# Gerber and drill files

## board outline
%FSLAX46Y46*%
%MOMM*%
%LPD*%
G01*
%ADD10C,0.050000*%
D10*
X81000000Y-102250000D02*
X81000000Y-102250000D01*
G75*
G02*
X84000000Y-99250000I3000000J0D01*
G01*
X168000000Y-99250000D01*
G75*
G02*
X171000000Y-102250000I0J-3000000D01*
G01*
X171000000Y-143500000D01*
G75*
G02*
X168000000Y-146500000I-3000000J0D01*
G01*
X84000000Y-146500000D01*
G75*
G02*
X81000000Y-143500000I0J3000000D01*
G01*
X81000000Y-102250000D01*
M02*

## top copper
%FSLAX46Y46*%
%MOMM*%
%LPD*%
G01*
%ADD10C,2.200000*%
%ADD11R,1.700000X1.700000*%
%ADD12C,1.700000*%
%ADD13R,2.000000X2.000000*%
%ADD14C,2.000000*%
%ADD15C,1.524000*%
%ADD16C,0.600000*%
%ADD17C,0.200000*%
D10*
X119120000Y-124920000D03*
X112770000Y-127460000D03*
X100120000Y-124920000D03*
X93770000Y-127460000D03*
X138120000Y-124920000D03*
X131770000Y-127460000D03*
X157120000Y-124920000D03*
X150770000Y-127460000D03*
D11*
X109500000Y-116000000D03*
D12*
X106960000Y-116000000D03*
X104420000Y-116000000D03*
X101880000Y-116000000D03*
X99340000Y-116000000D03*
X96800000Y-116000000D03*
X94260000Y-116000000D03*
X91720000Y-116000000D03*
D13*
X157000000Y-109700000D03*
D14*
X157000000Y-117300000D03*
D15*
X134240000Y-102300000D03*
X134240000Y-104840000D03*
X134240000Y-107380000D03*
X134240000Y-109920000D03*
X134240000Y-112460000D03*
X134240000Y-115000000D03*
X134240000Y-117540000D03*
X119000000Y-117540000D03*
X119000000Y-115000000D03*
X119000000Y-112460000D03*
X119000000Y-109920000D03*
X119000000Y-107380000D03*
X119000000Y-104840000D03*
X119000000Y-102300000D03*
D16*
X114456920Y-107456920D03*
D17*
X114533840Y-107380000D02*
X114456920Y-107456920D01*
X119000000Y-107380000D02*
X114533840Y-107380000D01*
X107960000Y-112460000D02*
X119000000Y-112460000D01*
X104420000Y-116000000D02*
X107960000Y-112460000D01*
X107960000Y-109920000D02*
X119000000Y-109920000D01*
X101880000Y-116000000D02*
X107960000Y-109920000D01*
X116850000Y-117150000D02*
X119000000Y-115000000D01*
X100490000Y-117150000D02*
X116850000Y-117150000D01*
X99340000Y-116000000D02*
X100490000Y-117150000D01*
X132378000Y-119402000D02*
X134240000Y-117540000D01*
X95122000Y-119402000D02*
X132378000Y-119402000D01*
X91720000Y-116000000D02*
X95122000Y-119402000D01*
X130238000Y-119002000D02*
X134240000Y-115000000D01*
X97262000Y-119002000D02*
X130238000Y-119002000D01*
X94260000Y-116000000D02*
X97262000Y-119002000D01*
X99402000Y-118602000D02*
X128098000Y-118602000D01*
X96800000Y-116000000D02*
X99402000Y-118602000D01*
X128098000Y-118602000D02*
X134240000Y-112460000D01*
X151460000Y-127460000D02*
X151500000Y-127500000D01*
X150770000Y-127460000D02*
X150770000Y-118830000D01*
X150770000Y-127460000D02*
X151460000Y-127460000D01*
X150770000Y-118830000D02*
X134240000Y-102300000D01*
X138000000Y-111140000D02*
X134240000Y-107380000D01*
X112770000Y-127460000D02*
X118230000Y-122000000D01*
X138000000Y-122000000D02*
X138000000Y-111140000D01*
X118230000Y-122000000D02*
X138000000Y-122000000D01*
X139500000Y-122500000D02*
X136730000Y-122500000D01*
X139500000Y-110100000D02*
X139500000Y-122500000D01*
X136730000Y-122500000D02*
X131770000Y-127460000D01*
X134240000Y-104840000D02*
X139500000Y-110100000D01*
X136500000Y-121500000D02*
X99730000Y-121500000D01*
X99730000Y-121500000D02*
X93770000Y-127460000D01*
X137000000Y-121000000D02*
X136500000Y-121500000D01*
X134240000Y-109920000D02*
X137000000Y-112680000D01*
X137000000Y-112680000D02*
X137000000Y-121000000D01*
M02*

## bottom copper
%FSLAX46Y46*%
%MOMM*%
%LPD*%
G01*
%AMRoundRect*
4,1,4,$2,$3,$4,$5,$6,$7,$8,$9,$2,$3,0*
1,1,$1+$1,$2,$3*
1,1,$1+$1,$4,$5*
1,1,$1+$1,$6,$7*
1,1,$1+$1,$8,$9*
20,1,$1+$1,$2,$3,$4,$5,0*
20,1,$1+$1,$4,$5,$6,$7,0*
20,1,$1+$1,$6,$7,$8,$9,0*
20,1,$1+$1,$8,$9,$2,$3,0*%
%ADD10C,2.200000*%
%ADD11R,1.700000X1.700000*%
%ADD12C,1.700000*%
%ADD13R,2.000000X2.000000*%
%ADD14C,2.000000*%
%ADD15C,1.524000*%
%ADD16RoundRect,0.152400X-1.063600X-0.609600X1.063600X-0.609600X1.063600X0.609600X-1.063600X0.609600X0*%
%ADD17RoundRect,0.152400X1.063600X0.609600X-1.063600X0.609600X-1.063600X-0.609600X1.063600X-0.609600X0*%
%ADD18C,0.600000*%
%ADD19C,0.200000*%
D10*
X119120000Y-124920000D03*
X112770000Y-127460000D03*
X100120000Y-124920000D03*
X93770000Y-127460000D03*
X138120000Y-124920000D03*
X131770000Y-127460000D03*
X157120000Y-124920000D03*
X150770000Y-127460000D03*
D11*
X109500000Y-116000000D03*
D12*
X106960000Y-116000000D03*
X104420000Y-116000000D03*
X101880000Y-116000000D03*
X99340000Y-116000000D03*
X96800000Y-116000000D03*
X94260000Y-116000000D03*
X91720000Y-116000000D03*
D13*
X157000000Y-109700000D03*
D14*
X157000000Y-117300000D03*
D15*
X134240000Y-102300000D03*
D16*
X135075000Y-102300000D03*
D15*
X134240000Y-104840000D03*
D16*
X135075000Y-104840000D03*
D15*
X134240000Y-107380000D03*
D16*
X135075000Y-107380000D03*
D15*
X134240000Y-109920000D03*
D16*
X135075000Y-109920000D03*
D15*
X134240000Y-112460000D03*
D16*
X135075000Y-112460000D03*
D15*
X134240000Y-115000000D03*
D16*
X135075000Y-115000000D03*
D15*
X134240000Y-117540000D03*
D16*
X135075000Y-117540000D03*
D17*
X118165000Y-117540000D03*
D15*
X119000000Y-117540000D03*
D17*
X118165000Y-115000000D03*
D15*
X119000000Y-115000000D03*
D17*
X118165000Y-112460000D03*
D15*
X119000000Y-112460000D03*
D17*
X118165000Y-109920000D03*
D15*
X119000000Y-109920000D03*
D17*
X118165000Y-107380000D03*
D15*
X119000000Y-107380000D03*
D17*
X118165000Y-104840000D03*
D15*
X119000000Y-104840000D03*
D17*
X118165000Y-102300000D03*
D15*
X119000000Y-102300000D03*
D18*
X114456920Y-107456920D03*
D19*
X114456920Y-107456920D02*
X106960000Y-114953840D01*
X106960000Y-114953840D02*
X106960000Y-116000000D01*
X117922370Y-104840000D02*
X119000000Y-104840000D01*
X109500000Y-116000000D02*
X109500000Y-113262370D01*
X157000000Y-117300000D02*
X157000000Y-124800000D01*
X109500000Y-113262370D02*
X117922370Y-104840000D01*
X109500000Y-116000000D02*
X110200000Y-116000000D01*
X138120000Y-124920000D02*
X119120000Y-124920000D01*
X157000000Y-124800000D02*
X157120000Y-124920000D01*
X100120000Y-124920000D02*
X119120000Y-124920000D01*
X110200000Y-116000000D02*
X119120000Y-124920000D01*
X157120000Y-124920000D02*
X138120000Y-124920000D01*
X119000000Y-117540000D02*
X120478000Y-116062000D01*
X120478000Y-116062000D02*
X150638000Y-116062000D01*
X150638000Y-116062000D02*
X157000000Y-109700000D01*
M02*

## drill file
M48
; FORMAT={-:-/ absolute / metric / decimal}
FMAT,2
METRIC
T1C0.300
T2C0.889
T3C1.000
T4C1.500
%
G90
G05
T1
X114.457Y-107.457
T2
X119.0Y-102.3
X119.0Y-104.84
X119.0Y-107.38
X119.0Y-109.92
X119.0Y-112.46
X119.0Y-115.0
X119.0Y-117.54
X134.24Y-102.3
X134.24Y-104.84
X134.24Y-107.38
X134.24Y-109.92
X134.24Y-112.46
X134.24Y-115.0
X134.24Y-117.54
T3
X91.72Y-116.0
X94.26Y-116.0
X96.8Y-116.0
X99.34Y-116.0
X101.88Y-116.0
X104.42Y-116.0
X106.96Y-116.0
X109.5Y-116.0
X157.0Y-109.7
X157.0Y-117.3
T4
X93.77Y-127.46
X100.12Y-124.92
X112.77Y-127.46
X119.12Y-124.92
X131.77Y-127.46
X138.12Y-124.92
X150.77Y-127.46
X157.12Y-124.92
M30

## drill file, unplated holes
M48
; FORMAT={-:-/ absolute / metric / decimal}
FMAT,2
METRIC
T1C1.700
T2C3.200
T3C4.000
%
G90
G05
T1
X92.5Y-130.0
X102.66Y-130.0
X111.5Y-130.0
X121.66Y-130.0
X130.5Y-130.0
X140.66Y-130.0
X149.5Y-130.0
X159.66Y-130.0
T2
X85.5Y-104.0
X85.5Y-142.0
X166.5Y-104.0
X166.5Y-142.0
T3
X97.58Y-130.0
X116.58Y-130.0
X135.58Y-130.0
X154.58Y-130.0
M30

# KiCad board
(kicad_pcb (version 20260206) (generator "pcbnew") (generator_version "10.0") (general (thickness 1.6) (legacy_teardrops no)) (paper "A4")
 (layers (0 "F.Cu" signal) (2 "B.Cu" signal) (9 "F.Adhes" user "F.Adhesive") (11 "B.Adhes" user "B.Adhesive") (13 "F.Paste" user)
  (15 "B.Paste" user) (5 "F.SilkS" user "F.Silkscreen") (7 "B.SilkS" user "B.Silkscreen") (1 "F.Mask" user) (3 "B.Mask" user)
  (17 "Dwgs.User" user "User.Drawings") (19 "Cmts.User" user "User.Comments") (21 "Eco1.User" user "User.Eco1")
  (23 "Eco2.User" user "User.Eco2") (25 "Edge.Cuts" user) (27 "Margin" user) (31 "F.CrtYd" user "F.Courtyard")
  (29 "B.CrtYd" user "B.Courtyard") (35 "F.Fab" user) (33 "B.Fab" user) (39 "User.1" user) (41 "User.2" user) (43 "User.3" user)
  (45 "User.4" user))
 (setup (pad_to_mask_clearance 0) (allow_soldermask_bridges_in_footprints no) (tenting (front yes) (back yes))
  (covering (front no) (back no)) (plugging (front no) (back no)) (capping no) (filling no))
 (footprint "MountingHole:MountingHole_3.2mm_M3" (layer "F.Cu") (at 85.5 104)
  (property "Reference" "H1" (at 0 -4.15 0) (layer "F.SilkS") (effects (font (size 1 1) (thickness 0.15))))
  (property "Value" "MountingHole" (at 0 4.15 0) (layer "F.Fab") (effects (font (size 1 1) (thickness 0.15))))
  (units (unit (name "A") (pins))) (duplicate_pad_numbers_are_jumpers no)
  (pad "" np_thru_hole circle (at 0 0) (size 3.2 3.2) (drill 3.2) (layers "*.Cu" "*.Mask")))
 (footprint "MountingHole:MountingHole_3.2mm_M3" (layer "F.Cu") (at 85.5 142)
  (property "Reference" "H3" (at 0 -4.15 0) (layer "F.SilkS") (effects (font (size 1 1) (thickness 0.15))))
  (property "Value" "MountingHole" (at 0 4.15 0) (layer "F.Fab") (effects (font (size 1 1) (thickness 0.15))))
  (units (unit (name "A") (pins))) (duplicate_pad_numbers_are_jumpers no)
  (pad "" np_thru_hole circle (at 0 0) (size 3.2 3.2) (drill 3.2) (layers "*.Cu" "*.Mask")))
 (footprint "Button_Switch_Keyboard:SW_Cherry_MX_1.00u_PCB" (layer "F.Cu") (at 119.12 124.92)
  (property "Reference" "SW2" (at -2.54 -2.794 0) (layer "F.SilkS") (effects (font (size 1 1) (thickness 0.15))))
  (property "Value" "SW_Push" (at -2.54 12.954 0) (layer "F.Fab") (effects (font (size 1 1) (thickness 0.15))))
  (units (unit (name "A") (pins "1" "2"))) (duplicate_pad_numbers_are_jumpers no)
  (pad "" np_thru_hole circle (at -7.62 5.08) (size 1.7 1.7) (drill 1.7) (layers "*.Cu" "*.Mask"))
  (pad "" np_thru_hole circle (at -2.54 5.08) (size 4 4) (drill 4) (layers "*.Cu" "*.Mask"))
  (pad "" np_thru_hole circle (at 2.54 5.08) (size 1.7 1.7) (drill 1.7) (layers "*.Cu" "*.Mask"))
  (pad "1" thru_hole circle (at 0 0) (size 2.2 2.2) (drill 1.5) (layers "*.Cu" "*.Mask") (remove_unused_layers no) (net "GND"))
  (pad "2" thru_hole circle (at -6.35 2.54) (size 2.2 2.2) (drill 1.5) (layers "*.Cu" "*.Mask") (remove_unused_layers no)
   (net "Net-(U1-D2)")))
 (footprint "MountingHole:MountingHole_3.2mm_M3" (layer "F.Cu") (at 166.5 142)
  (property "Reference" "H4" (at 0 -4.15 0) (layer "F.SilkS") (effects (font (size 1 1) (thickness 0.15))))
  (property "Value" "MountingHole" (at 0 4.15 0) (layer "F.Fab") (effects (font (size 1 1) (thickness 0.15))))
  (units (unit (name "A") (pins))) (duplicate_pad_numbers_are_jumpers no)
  (pad "" np_thru_hole circle (at 0 0) (size 3.2 3.2) (drill 3.2) (layers "*.Cu" "*.Mask")))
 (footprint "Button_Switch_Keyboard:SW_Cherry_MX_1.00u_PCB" (layer "F.Cu") (at 100.12 124.92)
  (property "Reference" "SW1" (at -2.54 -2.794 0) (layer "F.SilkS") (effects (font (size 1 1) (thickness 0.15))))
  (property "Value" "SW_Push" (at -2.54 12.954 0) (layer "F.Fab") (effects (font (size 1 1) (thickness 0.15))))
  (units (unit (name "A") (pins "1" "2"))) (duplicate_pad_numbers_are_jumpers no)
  (pad "" np_thru_hole circle (at -7.62 5.08) (size 1.7 1.7) (drill 1.7) (layers "*.Cu" "*.Mask"))
  (pad "" np_thru_hole circle (at -2.54 5.08) (size 4 4) (drill 4) (layers "*.Cu" "*.Mask"))
  (pad "" np_thru_hole circle (at 2.54 5.08) (size 1.7 1.7) (drill 1.7) (layers "*.Cu" "*.Mask"))
  (pad "1" thru_hole circle (at 0 0) (size 2.2 2.2) (drill 1.5) (layers "*.Cu" "*.Mask") (remove_unused_layers no) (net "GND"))
  (pad "2" thru_hole circle (at -6.35 2.54) (size 2.2 2.2) (drill 1.5) (layers "*.Cu" "*.Mask") (remove_unused_layers no)
   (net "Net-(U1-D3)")))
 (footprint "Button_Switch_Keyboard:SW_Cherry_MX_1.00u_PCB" (layer "F.Cu") (at 138.12 124.92)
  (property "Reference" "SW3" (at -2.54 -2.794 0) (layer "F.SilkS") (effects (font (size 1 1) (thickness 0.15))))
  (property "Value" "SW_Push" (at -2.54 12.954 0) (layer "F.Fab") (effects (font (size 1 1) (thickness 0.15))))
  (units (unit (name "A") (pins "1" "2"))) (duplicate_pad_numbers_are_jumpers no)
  (pad "" np_thru_hole circle (at -7.62 5.08) (size 1.7 1.7) (drill 1.7) (layers "*.Cu" "*.Mask"))
  (pad "" np_thru_hole circle (at -2.54 5.08) (size 4 4) (drill 4) (layers "*.Cu" "*.Mask"))
  (pad "" np_thru_hole circle (at 2.54 5.08) (size 1.7 1.7) (drill 1.7) (layers "*.Cu" "*.Mask"))
  (pad "1" thru_hole circle (at 0 0) (size 2.2 2.2) (drill 1.5) (layers "*.Cu" "*.Mask") (remove_unused_layers no) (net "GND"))
  (pad "2" thru_hole circle (at -6.35 2.54) (size 2.2 2.2) (drill 1.5) (layers "*.Cu" "*.Mask") (remove_unused_layers no)
   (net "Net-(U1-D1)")))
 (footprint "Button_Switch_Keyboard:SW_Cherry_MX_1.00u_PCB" (layer "F.Cu") (at 157.12 124.92)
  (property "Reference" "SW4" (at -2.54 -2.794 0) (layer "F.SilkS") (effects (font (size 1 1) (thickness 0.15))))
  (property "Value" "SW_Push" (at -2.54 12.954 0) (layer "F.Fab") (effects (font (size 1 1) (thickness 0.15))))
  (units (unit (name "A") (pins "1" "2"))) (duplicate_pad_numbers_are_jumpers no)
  (pad "" np_thru_hole circle (at -7.62 5.08) (size 1.7 1.7) (drill 1.7) (layers "*.Cu" "*.Mask"))
  (pad "" np_thru_hole circle (at -2.54 5.08) (size 4 4) (drill 4) (layers "*.Cu" "*.Mask"))
  (pad "" np_thru_hole circle (at 2.54 5.08) (size 1.7 1.7) (drill 1.7) (layers "*.Cu" "*.Mask"))
  (pad "1" thru_hole circle (at 0 0) (size 2.2 2.2) (drill 1.5) (layers "*.Cu" "*.Mask") (remove_unused_layers no) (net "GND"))
  (pad "2" thru_hole circle (at -6.35 2.54) (size 2.2 2.2) (drill 1.5) (layers "*.Cu" "*.Mask") (remove_unused_layers no)
   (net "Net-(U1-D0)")))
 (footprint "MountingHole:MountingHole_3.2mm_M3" (layer "F.Cu") (at 166.5 104)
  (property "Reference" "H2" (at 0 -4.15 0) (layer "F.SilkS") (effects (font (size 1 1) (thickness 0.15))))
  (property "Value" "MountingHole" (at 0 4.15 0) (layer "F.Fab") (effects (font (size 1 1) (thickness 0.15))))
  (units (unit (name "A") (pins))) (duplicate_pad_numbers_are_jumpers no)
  (pad "" np_thru_hole circle (at 0 0) (size 3.2 3.2) (drill 3.2) (layers "*.Cu" "*.Mask")))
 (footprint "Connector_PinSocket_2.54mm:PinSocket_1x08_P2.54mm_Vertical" (layer "B.Cu") (at 109.5 116 90)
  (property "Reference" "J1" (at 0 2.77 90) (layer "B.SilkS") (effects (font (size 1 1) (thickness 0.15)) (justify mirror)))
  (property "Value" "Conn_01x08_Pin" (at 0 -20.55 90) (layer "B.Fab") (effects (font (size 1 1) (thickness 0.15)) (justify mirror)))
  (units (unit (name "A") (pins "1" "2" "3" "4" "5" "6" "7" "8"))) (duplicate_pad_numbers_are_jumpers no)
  (pad "1" thru_hole rect (at 0 0 90) (size 1.7 1.7) (drill 1) (layers "*.Cu" "*.Mask") (remove_unused_layers no) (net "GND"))
  (pad "2" thru_hole circle (at 0 -2.54 90) (size 1.7 1.7) (drill 1) (layers "*.Cu" "*.Mask") (remove_unused_layers no) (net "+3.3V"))
  (pad "3" thru_hole circle (at 0 -5.08 90) (size 1.7 1.7) (drill 1) (layers "*.Cu" "*.Mask") (remove_unused_layers no) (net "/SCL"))
  (pad "4" thru_hole circle (at 0 -7.62 90) (size 1.7 1.7) (drill 1) (layers "*.Cu" "*.Mask") (remove_unused_layers no) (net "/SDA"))
  (pad "5" thru_hole circle (at 0 -10.16 90) (size 1.7 1.7) (drill 1) (layers "*.Cu" "*.Mask") (remove_unused_layers no) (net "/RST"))
  (pad "6" thru_hole circle (at 0 -12.7 90) (size 1.7 1.7) (drill 1) (layers "*.Cu" "*.Mask") (remove_unused_layers no) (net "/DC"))
  (pad "7" thru_hole circle (at 0 -15.24 90) (size 1.7 1.7) (drill 1) (layers "*.Cu" "*.Mask") (remove_unused_layers no) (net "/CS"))
  (pad "8" thru_hole circle (at 0 -17.78 90) (size 1.7 1.7) (drill 1) (layers "*.Cu" "*.Mask") (remove_unused_layers no) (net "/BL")))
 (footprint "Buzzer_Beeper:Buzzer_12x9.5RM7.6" (layer "B.Cu") (at 157 109.7 -90)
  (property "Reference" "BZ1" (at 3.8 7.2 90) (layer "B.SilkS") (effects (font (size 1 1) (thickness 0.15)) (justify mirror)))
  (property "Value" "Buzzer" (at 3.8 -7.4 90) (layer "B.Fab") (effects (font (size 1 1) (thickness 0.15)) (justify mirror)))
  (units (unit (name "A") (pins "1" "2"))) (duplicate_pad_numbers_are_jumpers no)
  (pad "1" thru_hole rect (at 0 0 270) (size 2 2) (drill 1) (layers "*.Cu" "*.Mask") (remove_unused_layers no) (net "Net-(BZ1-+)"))
  (pad "2" thru_hole circle (at 7.6 0 270) (size 2 2) (drill 1) (layers "*.Cu" "*.Mask") (remove_unused_layers no) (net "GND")))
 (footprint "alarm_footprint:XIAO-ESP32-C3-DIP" (layer "B.Cu") (at 126.62 109.92 90)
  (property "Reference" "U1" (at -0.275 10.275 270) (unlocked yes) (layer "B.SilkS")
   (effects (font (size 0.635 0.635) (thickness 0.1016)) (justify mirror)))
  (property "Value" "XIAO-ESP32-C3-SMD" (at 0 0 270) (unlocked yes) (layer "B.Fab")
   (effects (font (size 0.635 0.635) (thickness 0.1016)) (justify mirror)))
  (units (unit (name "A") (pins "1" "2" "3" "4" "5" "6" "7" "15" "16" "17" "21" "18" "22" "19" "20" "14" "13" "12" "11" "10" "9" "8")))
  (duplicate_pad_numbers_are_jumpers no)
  (pad "1" thru_hole circle (at 7.62 7.62) (size 1.524 1.524) (drill 0.889) (layers "*.Cu" "*.Mask") (remove_unused_layers no)
   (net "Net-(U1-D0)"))
  (pad "1" smd roundrect (at 7.62 8.455) (size 2.432 1.524) (layers "B.Cu" "B.Mask") (roundrect_rratio 0.1) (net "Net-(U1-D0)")
   (thermal_bridge_angle 45))
  (pad "2" thru_hole circle (at 5.08 7.62) (size 1.524 1.524) (drill 0.889) (layers "*.Cu" "*.Mask") (remove_unused_layers no)
   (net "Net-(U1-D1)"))
  (pad "2" smd roundrect (at 5.08 8.455) (size 2.432 1.524) (layers "B.Cu" "B.Mask") (roundrect_rratio 0.1) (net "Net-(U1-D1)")
   (thermal_bridge_angle 45))
  (pad "3" thru_hole circle (at 2.54 7.62) (size 1.524 1.524) (drill 0.889) (layers "*.Cu" "*.Mask") (remove_unused_layers no)
   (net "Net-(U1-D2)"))
  (pad "3" smd roundrect (at 2.54 8.455) (size 2.432 1.524) (layers "B.Cu" "B.Mask") (roundrect_rratio 0.1) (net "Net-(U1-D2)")
   (thermal_bridge_angle 45))
  (pad "4" thru_hole circle (at 0 7.62) (size 1.524 1.524) (drill 0.889) (layers "*.Cu" "*.Mask") (remove_unused_layers no)
   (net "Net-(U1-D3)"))
  (pad "4" smd roundrect (at 0 8.455) (size 2.432 1.524) (layers "B.Cu" "B.Mask") (roundrect_rratio 0.1) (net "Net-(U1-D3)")
   (thermal_bridge_angle 45))
  (pad "5" thru_hole circle (at -2.54 7.62) (size 1.524 1.524) (drill 0.889) (layers "*.Cu" "*.Mask") (remove_unused_layers no) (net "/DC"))
  (pad "5" smd roundrect (at -2.54 8.455) (size 2.432 1.524) (layers "B.Cu" "B.Mask") (roundrect_rratio 0.1) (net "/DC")
   (thermal_bridge_angle 45))
  (pad "6" thru_hole circle (at -5.08 7.62) (size 1.524 1.524) (drill 0.889) (layers "*.Cu" "*.Mask") (remove_unused_layers no) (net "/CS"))
  (pad "6" smd roundrect (at -5.08 8.455) (size 2.432 1.524) (layers "B.Cu" "B.Mask") (roundrect_rratio 0.1) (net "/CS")
   (thermal_bridge_angle 45))
  (pad "7" thru_hole circle (at -7.62 7.62) (size 1.524 1.524) (drill 0.889) (layers "*.Cu" "*.Mask") (remove_unused_layers no) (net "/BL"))
  (pad "7" smd roundrect (at -7.62 8.455) (size 2.432 1.524) (layers "B.Cu" "B.Mask") (roundrect_rratio 0.1) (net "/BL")
   (thermal_bridge_angle 45))
  (pad "8" smd roundrect (at -7.62 -8.455 180) (size 2.432 1.524) (layers "B.Cu" "B.Mask") (roundrect_rratio 0.1) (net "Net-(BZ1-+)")
   (thermal_bridge_angle 45))
  (pad "8" thru_hole circle (at -7.62 -7.62 180) (size 1.524 1.524) (drill 0.889) (layers "*.Cu" "*.Mask") (remove_unused_layers no)
   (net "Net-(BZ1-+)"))
  (pad "9" smd roundrect (at -5.08 -8.455 180) (size 2.432 1.524) (layers "B.Cu" "B.Mask") (roundrect_rratio 0.1) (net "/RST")
   (thermal_bridge_angle 45))
  (pad "9" thru_hole circle (at -5.08 -7.62 180) (size 1.524 1.524) (drill 0.889) (layers "*.Cu" "*.Mask") (remove_unused_layers no)
   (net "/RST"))
  (pad "10" smd roundrect (at -2.54 -8.455 180) (size 2.432 1.524) (layers "B.Cu" "B.Mask") (roundrect_rratio 0.1) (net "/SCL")
   (thermal_bridge_angle 45))
  (pad "10" thru_hole circle (at -2.54 -7.62 180) (size 1.524 1.524) (drill 0.889) (layers "*.Cu" "*.Mask") (remove_unused_layers no)
   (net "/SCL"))
  (pad "11" smd roundrect (at 0 -8.455 180) (size 2.432 1.524) (layers "B.Cu" "B.Mask") (roundrect_rratio 0.1) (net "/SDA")
   (thermal_bridge_angle 45))
  (pad "11" thru_hole circle (at 0 -7.62 180) (size 1.524 1.524) (drill 0.889) (layers "*.Cu" "*.Mask") (remove_unused_layers no)
   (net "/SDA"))
  (pad "12" smd roundrect (at 2.54 -8.455 180) (size 2.432 1.524) (layers "B.Cu" "B.Mask") (roundrect_rratio 0.1) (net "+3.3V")
   (thermal_bridge_angle 45))
  (pad "12" thru_hole circle (at 2.54 -7.62 180) (size 1.524 1.524) (drill 0.889) (layers "*.Cu" "*.Mask") (remove_unused_layers no)
   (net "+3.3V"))
  (pad "13" smd roundrect (at 5.08 -8.455 180) (size 2.432 1.524) (layers "B.Cu" "B.Mask") (roundrect_rratio 0.1) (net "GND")
   (thermal_bridge_angle 45))
  (pad "13" thru_hole circle (at 5.08 -7.62 180) (size 1.524 1.524) (drill 0.889) (layers "*.Cu" "*.Mask") (remove_unused_layers no)
   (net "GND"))
  (pad "14" smd roundrect (at 7.62 -8.455 180) (size 2.432 1.524) (layers "B.Cu" "B.Mask") (roundrect_rratio 0.1)
   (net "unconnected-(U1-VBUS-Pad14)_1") (thermal_bridge_angle 45))
  (pad "14" thru_hole circle (at 7.62 -7.62 180) (size 1.524 1.524) (drill 0.889) (layers "*.Cu" "*.Mask") (remove_unused_layers no)
   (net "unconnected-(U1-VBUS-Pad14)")))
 (gr_rect (start 81 99.25) (end 171 146.5) (radius 3) (stroke (width 0.05) (type solid)) (fill no) (layer "Edge.Cuts"))
 (segment (start 117.92237 104.84) (end 119 104.84) (width 0.2) (layer "B.Cu") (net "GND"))
 (segment (start 109.5 116) (end 109.5 113.26237) (width 0.2) (layer "B.Cu") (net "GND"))
 (segment (start 157 117.3) (end 157 124.8) (width 0.2) (layer "B.Cu") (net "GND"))
 (segment (start 109.5 113.26237) (end 117.92237 104.84) (width 0.2) (layer "B.Cu") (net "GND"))
 (segment (start 109.5 116) (end 110.2 116) (width 0.2) (layer "B.Cu") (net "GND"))
 (segment (start 138.12 124.92) (end 119.12 124.92) (width 0.2) (layer "B.Cu") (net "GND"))
 (segment (start 157 124.8) (end 157.12 124.92) (width 0.2) (layer "B.Cu") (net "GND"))
 (segment (start 100.12 124.92) (end 119.12 124.92) (width 0.2) (layer "B.Cu") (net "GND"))
 (segment (start 110.2 116) (end 119.12 124.92) (width 0.2) (layer "B.Cu") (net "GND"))
 (segment (start 157.12 124.92) (end 138.12 124.92) (width 0.2) (layer "B.Cu") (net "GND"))
 (segment (start 138 111.14) (end 134.24 107.38) (width 0.2) (layer "F.Cu") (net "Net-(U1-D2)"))
 (segment (start 112.77 127.46) (end 118.23 122) (width 0.2) (layer "F.Cu") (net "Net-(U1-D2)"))
 (segment (start 138 122) (end 138 111.14) (width 0.2) (layer "F.Cu") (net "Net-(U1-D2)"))
 (segment (start 118.23 122) (end 138 122) (width 0.2) (layer "F.Cu") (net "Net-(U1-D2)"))
 (segment (start 136.5 121.5) (end 99.73 121.5) (width 0.2) (layer "F.Cu") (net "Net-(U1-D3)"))
 (segment (start 99.73 121.5) (end 93.77 127.46) (width 0.2) (layer "F.Cu") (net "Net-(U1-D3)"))
 (segment (start 137 121) (end 136.5 121.5) (width 0.2) (layer "F.Cu") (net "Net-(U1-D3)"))
 (segment (start 134.24 109.92) (end 137 112.68) (width 0.2) (layer "F.Cu") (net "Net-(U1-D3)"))
 (segment (start 137 112.68) (end 137 121) (width 0.2) (layer "F.Cu") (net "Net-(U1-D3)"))
 (segment (start 139.5 122.5) (end 136.73 122.5) (width 0.2) (layer "F.Cu") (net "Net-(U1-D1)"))
 (segment (start 139.5 110.1) (end 139.5 122.5) (width 0.2) (layer "F.Cu") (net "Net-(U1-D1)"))
 (segment (start 136.73 122.5) (end 131.77 127.46) (width 0.2) (layer "F.Cu") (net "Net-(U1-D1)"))
 (segment (start 134.24 104.84) (end 139.5 110.1) (width 0.2) (layer "F.Cu") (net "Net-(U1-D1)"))
 (segment (start 151.46 127.46) (end 151.5 127.5) (width 0.2) (layer "F.Cu") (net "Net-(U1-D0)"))
 (segment (start 150.77 127.46) (end 150.77 118.83) (width 0.2) (layer "F.Cu") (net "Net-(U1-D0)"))
 (segment (start 150.77 127.46) (end 151.46 127.46) (width 0.2) (layer "F.Cu") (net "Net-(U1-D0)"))
 (segment (start 150.77 118.83) (end 134.24 102.3) (width 0.2) (layer "F.Cu") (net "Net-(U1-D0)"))
 (segment (start 119 107.38) (end 114.53384 107.38) (width 0.2) (layer "F.Cu") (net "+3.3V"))
 (segment (start 114.53384 107.38) (end 114.45692 107.45692) (width 0.2) (layer "F.Cu") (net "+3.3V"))
 (via (at 114.45692 107.45692) (size 0.6) (drill 0.3) (layers "F.Cu" "B.Cu") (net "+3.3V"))
 (segment (start 106.96 114.95384) (end 106.96 116) (width 0.2) (layer "B.Cu") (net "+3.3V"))
 (segment (start 114.45692 107.45692) (end 106.96 114.95384) (width 0.2) (layer "B.Cu") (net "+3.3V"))
 (segment (start 107.96 112.46) (end 119 112.46) (width 0.2) (layer "F.Cu") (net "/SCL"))
 (segment (start 104.42 116) (end 107.96 112.46) (width 0.2) (layer "F.Cu") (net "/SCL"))
 (segment (start 107.96 109.92) (end 119 109.92) (width 0.2) (layer "F.Cu") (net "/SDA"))
 (segment (start 101.88 116) (end 107.96 109.92) (width 0.2) (layer "F.Cu") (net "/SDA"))
 (segment (start 100.49 117.15) (end 116.85 117.15) (width 0.2) (layer "F.Cu") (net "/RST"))
 (segment (start 99.34 116) (end 100.49 117.15) (width 0.2) (layer "F.Cu") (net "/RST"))
 (segment (start 116.85 117.15) (end 119 115) (width 0.2) (layer "F.Cu") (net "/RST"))
 (segment (start 128.098 118.602) (end 134.24 112.46) (width 0.2) (layer "F.Cu") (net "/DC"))
 (segment (start 96.8 116) (end 99.402 118.602) (width 0.2) (layer "F.Cu") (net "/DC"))
 (segment (start 99.402 118.602) (end 128.098 118.602) (width 0.2) (layer "F.Cu") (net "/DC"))
 (segment (start 130.238 119.002) (end 134.24 115) (width 0.2) (layer "F.Cu") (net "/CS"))
 (segment (start 97.262 119.002) (end 130.238 119.002) (width 0.2) (layer "F.Cu") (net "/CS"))
 (segment (start 94.26 116) (end 97.262 119.002) (width 0.2) (layer "F.Cu") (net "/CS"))
 (segment (start 95.122 119.402) (end 132.378 119.402) (width 0.2) (layer "F.Cu") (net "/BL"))
 (segment (start 91.72 116) (end 95.122 119.402) (width 0.2) (layer "F.Cu") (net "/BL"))
 (segment (start 132.378 119.402) (end 134.24 117.54) (width 0.2) (layer "F.Cu") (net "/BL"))
 (segment (start 119 117.54) (end 120.478 116.062) (width 0.2) (layer "B.Cu") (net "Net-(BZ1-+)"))
 (segment (start 120.478 116.062) (end 150.638 116.062) (width 0.2) (layer "B.Cu") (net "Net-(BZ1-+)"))
 (segment (start 150.638 116.062) (end 157 109.7) (width 0.2) (layer "B.Cu") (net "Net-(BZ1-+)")))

